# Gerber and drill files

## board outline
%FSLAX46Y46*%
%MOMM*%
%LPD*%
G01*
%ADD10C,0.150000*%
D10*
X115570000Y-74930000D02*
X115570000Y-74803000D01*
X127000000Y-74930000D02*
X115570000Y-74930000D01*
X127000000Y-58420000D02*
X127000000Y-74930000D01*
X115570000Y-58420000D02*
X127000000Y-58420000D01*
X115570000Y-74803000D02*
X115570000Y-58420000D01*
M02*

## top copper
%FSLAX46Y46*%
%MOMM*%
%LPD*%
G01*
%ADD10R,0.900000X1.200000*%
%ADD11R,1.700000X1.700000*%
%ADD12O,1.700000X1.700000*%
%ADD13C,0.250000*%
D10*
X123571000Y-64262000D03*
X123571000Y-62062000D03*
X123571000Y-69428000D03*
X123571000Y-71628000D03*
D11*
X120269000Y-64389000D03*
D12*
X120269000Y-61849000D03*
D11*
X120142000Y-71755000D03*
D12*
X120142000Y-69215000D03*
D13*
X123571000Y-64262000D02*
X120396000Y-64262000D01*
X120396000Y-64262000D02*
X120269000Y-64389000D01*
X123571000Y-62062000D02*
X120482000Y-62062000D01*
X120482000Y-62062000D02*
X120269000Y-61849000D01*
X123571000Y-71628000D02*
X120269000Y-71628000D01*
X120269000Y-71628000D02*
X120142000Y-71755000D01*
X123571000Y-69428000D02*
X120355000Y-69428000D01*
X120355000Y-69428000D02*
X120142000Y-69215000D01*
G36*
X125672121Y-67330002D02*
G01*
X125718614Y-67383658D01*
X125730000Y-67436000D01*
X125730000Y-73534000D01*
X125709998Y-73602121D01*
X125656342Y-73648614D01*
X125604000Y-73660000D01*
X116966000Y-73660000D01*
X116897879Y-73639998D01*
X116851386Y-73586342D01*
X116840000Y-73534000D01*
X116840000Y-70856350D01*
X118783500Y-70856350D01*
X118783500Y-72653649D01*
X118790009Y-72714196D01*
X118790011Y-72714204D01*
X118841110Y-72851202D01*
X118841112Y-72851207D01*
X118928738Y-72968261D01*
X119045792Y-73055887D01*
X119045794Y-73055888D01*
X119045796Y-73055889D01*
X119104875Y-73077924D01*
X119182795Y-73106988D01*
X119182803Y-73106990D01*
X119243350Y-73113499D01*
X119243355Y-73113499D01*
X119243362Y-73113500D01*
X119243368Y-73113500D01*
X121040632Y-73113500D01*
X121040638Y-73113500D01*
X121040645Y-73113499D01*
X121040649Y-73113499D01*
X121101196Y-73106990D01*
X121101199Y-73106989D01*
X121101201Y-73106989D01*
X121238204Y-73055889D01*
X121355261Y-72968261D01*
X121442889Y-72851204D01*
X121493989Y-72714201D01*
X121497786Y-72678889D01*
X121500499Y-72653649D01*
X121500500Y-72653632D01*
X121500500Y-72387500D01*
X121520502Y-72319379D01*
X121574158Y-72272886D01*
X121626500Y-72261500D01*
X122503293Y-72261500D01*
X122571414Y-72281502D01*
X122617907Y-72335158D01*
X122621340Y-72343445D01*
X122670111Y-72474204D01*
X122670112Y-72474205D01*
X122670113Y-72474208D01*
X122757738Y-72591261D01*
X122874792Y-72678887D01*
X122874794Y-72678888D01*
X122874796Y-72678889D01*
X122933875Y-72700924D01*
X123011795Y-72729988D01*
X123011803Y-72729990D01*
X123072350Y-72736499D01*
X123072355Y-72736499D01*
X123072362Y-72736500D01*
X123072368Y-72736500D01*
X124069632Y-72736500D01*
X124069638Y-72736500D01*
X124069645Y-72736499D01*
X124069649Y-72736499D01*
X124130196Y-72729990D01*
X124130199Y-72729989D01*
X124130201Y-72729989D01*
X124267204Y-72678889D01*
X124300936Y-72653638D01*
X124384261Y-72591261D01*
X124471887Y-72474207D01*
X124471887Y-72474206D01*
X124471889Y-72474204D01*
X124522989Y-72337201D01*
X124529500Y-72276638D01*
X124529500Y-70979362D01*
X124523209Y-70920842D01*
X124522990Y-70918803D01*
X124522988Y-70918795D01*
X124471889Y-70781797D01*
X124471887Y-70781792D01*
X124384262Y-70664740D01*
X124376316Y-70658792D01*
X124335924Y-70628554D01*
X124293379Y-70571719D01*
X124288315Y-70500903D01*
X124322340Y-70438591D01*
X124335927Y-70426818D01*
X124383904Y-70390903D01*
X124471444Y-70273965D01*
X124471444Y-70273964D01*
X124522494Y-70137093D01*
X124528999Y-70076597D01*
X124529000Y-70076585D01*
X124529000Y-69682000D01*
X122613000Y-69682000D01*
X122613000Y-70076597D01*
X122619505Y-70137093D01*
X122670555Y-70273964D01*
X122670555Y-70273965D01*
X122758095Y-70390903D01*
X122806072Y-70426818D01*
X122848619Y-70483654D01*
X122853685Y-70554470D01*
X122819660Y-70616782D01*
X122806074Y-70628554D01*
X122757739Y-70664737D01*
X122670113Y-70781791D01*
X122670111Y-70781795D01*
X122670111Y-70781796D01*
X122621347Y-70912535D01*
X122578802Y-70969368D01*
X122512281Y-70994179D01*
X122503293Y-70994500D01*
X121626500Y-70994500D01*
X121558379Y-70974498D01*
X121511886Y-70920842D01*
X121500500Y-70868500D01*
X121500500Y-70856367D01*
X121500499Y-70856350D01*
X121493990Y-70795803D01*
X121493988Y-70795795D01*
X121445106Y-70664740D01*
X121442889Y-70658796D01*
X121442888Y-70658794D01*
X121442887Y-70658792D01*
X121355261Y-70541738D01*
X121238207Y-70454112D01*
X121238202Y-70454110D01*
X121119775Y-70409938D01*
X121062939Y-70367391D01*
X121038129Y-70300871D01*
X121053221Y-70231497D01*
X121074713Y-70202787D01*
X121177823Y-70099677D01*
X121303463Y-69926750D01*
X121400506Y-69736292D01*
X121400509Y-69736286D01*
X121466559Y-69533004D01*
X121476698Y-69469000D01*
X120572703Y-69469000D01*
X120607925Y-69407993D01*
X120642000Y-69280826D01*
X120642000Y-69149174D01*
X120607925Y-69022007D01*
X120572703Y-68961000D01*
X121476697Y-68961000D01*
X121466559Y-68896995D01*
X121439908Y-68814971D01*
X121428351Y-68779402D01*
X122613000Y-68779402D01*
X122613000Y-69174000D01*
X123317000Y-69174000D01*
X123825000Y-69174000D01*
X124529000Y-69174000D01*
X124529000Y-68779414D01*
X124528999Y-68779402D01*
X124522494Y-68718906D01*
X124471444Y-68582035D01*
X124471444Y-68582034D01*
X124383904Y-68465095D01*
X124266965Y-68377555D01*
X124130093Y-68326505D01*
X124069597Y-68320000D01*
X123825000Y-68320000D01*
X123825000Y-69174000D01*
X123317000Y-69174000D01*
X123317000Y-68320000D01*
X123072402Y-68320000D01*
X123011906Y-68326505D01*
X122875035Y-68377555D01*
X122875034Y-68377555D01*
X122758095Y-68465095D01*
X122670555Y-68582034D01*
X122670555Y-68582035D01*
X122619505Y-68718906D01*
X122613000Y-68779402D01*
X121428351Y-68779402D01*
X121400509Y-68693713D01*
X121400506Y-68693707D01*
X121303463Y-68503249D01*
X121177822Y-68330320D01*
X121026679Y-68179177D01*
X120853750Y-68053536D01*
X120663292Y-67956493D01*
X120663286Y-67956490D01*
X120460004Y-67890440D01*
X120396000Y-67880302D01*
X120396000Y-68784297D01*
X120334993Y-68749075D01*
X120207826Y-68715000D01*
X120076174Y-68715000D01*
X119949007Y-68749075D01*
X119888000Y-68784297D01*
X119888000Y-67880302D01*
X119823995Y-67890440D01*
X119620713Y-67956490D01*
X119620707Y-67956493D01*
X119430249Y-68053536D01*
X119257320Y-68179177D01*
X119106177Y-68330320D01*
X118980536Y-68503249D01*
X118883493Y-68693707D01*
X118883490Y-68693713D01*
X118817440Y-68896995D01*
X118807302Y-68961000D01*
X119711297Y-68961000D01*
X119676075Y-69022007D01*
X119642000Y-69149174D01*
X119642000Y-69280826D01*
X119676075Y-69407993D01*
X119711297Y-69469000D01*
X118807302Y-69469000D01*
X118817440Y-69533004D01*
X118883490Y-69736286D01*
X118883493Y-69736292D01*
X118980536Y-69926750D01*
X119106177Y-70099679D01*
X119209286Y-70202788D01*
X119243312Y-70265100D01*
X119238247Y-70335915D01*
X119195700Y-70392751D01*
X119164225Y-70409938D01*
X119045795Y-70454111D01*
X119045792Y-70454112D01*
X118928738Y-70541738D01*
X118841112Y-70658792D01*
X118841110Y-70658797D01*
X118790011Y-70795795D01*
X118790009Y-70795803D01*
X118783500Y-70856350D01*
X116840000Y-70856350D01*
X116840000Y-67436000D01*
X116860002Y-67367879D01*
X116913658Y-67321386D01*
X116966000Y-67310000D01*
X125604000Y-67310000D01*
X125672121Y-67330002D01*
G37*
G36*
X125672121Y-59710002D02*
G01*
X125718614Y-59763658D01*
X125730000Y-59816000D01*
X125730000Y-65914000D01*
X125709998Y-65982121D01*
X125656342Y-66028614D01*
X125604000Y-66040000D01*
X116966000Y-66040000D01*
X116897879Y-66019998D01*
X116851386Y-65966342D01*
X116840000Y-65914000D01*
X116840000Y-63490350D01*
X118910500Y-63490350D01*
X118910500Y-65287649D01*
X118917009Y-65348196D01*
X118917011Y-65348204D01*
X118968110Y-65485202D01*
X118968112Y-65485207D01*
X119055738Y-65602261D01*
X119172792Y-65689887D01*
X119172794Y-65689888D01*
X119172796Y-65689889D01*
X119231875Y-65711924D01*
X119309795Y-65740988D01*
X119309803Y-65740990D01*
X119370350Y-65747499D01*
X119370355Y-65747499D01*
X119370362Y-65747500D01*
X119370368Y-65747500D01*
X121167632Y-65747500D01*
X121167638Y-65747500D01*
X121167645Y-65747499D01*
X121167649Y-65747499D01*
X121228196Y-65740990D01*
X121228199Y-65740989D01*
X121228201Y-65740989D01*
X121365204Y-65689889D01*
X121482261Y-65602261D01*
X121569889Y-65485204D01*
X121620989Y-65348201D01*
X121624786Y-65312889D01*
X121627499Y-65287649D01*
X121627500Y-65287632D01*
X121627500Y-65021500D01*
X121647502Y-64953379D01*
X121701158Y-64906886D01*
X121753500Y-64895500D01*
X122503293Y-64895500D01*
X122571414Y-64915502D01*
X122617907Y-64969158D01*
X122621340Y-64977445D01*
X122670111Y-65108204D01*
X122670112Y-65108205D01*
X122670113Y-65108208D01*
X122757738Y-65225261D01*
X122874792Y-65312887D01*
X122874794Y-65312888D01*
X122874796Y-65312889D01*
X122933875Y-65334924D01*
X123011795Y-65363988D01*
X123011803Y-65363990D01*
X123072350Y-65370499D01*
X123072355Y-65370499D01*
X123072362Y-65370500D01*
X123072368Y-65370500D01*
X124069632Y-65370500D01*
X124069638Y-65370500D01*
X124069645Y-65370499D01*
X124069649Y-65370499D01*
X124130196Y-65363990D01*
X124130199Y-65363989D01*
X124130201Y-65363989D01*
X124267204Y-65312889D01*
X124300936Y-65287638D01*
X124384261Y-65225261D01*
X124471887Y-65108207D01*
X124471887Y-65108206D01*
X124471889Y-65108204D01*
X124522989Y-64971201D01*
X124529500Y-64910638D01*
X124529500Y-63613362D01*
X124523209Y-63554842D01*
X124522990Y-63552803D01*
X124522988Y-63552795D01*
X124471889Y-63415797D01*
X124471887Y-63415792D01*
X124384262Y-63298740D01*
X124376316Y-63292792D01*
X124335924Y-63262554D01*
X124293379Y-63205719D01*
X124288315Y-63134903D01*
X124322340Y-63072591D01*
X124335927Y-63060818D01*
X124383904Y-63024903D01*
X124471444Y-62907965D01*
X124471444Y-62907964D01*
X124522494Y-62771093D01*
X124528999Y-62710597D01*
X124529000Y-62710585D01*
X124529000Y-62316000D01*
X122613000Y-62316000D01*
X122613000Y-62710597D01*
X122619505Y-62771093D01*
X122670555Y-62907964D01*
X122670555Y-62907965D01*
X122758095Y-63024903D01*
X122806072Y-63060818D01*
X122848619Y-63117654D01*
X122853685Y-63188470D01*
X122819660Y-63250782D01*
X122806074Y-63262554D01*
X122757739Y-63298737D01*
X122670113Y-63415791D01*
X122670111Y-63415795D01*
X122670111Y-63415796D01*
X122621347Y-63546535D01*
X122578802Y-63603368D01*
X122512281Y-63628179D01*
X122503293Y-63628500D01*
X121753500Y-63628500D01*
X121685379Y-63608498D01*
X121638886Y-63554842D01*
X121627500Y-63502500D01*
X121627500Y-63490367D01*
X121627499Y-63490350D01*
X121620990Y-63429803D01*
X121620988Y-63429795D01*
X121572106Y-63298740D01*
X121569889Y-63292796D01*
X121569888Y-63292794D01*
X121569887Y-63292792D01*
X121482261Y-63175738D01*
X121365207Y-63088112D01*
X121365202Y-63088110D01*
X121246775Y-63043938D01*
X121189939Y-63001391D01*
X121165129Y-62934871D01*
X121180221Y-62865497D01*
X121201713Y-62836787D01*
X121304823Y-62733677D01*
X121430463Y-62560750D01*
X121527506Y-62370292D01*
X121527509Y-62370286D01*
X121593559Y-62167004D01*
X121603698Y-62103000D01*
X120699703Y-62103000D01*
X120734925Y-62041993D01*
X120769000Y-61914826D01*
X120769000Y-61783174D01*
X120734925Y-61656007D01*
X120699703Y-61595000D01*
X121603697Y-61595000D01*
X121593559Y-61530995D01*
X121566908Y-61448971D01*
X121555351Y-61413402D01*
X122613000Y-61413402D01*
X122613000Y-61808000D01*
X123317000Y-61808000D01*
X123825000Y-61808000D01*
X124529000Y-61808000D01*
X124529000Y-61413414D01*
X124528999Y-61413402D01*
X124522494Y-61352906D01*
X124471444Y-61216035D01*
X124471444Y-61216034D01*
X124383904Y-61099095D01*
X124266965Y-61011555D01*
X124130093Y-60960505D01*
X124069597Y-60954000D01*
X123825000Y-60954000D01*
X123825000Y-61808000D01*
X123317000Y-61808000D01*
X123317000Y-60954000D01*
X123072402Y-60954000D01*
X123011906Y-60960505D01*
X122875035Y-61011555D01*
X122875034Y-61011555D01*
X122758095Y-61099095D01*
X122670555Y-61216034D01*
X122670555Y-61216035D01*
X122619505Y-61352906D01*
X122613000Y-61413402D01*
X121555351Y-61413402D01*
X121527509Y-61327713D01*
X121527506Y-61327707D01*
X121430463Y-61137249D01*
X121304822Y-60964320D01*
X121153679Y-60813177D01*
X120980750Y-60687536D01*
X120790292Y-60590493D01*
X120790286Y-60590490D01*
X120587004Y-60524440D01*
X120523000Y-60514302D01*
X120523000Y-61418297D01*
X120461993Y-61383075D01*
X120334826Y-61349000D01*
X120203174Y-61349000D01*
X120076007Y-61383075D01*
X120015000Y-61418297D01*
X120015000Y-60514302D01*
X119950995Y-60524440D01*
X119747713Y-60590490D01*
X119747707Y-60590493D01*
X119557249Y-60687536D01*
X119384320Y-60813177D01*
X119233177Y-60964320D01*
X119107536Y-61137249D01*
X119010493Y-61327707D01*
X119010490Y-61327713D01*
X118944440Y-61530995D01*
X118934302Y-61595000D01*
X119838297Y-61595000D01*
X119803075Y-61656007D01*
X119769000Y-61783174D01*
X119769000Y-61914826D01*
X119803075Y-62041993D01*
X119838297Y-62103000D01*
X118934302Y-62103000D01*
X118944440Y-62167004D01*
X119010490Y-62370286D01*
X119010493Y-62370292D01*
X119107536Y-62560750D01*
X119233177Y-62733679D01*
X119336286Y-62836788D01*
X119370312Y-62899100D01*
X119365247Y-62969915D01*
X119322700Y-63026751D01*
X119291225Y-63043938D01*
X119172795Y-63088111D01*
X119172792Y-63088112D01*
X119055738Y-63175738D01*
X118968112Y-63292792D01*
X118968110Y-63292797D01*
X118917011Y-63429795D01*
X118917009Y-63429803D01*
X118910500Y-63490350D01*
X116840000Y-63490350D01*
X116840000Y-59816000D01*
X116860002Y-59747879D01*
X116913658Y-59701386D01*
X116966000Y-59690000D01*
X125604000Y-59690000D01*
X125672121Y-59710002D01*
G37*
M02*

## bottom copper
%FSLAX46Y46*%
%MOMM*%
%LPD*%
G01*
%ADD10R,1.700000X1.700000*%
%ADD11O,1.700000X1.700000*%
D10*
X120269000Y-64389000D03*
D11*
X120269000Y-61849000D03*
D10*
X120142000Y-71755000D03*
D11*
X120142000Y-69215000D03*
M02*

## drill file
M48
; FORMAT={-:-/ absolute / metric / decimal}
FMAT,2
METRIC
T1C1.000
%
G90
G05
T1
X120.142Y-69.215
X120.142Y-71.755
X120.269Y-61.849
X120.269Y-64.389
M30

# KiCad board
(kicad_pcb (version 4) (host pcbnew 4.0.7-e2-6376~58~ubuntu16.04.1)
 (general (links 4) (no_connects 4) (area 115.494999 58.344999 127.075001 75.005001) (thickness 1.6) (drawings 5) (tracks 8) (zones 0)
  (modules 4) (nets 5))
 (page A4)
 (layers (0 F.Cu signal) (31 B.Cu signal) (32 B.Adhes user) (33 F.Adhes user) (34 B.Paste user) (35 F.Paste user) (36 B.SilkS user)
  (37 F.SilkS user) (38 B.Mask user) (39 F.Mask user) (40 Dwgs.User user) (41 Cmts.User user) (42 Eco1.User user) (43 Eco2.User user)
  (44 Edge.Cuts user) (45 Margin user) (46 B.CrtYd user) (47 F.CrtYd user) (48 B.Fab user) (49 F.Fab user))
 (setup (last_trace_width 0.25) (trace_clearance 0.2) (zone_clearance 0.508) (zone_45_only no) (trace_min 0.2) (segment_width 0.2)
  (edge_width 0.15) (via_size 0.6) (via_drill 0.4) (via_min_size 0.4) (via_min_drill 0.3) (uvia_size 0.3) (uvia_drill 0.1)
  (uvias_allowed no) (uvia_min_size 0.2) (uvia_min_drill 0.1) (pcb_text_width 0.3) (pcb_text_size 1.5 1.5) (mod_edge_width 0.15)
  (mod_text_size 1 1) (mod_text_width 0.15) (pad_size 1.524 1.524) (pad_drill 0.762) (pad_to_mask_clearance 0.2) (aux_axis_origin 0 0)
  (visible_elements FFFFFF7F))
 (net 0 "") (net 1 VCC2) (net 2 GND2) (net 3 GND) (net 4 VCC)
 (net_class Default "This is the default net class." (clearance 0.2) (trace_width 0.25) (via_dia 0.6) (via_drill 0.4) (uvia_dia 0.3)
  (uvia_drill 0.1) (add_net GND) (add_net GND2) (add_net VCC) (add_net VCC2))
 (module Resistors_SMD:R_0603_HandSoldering (layer F.Cu) (at 123.571 63.162 90)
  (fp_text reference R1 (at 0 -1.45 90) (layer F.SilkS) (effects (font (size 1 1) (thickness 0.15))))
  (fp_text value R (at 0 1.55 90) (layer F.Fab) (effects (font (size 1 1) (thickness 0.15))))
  (pad 1 smd rect (at -1.1 0 90) (size 1.2 0.9) (layers F.Cu F.Paste F.Mask) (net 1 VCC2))
  (pad 2 smd rect (at 1.1 0 90) (size 1.2 0.9) (layers F.Cu F.Paste F.Mask) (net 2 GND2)))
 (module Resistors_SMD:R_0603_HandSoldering (layer F.Cu) (at 123.571 70.528 270)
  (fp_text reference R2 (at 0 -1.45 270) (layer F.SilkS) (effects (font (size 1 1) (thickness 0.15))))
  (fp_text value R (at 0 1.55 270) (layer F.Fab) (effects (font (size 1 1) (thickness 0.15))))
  (pad 1 smd rect (at -1.1 0 270) (size 1.2 0.9) (layers F.Cu F.Paste F.Mask) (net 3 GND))
  (pad 2 smd rect (at 1.1 0 270) (size 1.2 0.9) (layers F.Cu F.Paste F.Mask) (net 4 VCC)))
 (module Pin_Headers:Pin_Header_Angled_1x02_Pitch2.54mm (layer F.Cu) (at 120.269 64.389 180)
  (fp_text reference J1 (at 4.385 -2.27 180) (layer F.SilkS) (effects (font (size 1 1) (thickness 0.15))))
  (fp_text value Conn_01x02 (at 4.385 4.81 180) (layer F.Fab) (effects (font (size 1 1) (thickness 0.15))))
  (pad 1 thru_hole rect (at 0 0 180) (size 1.7 1.7) (drill 1) (layers *.Cu *.Mask) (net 1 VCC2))
  (pad 2 thru_hole oval (at 0 2.54 180) (size 1.7 1.7) (drill 1) (layers *.Cu *.Mask) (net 2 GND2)))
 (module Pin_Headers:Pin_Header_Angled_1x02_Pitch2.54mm (layer F.Cu) (at 120.142 71.755 180)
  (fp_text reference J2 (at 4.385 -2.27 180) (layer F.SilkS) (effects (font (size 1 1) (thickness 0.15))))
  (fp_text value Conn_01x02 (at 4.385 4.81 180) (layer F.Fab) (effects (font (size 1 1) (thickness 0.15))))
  (pad 1 thru_hole rect (at 0 0 180) (size 1.7 1.7) (drill 1) (layers *.Cu *.Mask) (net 4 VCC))
  (pad 2 thru_hole oval (at 0 2.54 180) (size 1.7 1.7) (drill 1) (layers *.Cu *.Mask) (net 3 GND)))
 (gr_line (start 115.57 74.93) (end 115.57 74.803) (layer Edge.Cuts) (width 0.15))
 (gr_line (start 127 74.93) (end 115.57 74.93) (layer Edge.Cuts) (width 0.15))
 (gr_line (start 127 58.42) (end 127 74.93) (layer Edge.Cuts) (width 0.15))
 (gr_line (start 115.57 58.42) (end 127 58.42) (layer Edge.Cuts) (width 0.15))
 (gr_line (start 115.57 74.803) (end 115.57 58.42) (layer Edge.Cuts) (width 0.15))
 (segment (start 123.571 64.262) (end 120.396 64.262) (width 0.25) (layer F.Cu) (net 1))
 (segment (start 120.396 64.262) (end 120.269 64.389) (width 0.25) (layer F.Cu) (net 1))
 (segment (start 123.571 62.062) (end 120.482 62.062) (width 0.25) (layer F.Cu) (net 2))
 (segment (start 120.482 62.062) (end 120.269 61.849) (width 0.25) (layer F.Cu) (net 2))
 (segment (start 123.571 71.628) (end 120.269 71.628) (width 0.25) (layer F.Cu) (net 4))
 (segment (start 120.269 71.628) (end 120.142 71.755) (width 0.25) (layer F.Cu) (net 4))
 (segment (start 123.571 69.428) (end 120.355 69.428) (width 0.25) (layer F.Cu) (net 3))
 (segment (start 120.355 69.428) (end 120.142 69.215) (width 0.25) (layer F.Cu) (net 3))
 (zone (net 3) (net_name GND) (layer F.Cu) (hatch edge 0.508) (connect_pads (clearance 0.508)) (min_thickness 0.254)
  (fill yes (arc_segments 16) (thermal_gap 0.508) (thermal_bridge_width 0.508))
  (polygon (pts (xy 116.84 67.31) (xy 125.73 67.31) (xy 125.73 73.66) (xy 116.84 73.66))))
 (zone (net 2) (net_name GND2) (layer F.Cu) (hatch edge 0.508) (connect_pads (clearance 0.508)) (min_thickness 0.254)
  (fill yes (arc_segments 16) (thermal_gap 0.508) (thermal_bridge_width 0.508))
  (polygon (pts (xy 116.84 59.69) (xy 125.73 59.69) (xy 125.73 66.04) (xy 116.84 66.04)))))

